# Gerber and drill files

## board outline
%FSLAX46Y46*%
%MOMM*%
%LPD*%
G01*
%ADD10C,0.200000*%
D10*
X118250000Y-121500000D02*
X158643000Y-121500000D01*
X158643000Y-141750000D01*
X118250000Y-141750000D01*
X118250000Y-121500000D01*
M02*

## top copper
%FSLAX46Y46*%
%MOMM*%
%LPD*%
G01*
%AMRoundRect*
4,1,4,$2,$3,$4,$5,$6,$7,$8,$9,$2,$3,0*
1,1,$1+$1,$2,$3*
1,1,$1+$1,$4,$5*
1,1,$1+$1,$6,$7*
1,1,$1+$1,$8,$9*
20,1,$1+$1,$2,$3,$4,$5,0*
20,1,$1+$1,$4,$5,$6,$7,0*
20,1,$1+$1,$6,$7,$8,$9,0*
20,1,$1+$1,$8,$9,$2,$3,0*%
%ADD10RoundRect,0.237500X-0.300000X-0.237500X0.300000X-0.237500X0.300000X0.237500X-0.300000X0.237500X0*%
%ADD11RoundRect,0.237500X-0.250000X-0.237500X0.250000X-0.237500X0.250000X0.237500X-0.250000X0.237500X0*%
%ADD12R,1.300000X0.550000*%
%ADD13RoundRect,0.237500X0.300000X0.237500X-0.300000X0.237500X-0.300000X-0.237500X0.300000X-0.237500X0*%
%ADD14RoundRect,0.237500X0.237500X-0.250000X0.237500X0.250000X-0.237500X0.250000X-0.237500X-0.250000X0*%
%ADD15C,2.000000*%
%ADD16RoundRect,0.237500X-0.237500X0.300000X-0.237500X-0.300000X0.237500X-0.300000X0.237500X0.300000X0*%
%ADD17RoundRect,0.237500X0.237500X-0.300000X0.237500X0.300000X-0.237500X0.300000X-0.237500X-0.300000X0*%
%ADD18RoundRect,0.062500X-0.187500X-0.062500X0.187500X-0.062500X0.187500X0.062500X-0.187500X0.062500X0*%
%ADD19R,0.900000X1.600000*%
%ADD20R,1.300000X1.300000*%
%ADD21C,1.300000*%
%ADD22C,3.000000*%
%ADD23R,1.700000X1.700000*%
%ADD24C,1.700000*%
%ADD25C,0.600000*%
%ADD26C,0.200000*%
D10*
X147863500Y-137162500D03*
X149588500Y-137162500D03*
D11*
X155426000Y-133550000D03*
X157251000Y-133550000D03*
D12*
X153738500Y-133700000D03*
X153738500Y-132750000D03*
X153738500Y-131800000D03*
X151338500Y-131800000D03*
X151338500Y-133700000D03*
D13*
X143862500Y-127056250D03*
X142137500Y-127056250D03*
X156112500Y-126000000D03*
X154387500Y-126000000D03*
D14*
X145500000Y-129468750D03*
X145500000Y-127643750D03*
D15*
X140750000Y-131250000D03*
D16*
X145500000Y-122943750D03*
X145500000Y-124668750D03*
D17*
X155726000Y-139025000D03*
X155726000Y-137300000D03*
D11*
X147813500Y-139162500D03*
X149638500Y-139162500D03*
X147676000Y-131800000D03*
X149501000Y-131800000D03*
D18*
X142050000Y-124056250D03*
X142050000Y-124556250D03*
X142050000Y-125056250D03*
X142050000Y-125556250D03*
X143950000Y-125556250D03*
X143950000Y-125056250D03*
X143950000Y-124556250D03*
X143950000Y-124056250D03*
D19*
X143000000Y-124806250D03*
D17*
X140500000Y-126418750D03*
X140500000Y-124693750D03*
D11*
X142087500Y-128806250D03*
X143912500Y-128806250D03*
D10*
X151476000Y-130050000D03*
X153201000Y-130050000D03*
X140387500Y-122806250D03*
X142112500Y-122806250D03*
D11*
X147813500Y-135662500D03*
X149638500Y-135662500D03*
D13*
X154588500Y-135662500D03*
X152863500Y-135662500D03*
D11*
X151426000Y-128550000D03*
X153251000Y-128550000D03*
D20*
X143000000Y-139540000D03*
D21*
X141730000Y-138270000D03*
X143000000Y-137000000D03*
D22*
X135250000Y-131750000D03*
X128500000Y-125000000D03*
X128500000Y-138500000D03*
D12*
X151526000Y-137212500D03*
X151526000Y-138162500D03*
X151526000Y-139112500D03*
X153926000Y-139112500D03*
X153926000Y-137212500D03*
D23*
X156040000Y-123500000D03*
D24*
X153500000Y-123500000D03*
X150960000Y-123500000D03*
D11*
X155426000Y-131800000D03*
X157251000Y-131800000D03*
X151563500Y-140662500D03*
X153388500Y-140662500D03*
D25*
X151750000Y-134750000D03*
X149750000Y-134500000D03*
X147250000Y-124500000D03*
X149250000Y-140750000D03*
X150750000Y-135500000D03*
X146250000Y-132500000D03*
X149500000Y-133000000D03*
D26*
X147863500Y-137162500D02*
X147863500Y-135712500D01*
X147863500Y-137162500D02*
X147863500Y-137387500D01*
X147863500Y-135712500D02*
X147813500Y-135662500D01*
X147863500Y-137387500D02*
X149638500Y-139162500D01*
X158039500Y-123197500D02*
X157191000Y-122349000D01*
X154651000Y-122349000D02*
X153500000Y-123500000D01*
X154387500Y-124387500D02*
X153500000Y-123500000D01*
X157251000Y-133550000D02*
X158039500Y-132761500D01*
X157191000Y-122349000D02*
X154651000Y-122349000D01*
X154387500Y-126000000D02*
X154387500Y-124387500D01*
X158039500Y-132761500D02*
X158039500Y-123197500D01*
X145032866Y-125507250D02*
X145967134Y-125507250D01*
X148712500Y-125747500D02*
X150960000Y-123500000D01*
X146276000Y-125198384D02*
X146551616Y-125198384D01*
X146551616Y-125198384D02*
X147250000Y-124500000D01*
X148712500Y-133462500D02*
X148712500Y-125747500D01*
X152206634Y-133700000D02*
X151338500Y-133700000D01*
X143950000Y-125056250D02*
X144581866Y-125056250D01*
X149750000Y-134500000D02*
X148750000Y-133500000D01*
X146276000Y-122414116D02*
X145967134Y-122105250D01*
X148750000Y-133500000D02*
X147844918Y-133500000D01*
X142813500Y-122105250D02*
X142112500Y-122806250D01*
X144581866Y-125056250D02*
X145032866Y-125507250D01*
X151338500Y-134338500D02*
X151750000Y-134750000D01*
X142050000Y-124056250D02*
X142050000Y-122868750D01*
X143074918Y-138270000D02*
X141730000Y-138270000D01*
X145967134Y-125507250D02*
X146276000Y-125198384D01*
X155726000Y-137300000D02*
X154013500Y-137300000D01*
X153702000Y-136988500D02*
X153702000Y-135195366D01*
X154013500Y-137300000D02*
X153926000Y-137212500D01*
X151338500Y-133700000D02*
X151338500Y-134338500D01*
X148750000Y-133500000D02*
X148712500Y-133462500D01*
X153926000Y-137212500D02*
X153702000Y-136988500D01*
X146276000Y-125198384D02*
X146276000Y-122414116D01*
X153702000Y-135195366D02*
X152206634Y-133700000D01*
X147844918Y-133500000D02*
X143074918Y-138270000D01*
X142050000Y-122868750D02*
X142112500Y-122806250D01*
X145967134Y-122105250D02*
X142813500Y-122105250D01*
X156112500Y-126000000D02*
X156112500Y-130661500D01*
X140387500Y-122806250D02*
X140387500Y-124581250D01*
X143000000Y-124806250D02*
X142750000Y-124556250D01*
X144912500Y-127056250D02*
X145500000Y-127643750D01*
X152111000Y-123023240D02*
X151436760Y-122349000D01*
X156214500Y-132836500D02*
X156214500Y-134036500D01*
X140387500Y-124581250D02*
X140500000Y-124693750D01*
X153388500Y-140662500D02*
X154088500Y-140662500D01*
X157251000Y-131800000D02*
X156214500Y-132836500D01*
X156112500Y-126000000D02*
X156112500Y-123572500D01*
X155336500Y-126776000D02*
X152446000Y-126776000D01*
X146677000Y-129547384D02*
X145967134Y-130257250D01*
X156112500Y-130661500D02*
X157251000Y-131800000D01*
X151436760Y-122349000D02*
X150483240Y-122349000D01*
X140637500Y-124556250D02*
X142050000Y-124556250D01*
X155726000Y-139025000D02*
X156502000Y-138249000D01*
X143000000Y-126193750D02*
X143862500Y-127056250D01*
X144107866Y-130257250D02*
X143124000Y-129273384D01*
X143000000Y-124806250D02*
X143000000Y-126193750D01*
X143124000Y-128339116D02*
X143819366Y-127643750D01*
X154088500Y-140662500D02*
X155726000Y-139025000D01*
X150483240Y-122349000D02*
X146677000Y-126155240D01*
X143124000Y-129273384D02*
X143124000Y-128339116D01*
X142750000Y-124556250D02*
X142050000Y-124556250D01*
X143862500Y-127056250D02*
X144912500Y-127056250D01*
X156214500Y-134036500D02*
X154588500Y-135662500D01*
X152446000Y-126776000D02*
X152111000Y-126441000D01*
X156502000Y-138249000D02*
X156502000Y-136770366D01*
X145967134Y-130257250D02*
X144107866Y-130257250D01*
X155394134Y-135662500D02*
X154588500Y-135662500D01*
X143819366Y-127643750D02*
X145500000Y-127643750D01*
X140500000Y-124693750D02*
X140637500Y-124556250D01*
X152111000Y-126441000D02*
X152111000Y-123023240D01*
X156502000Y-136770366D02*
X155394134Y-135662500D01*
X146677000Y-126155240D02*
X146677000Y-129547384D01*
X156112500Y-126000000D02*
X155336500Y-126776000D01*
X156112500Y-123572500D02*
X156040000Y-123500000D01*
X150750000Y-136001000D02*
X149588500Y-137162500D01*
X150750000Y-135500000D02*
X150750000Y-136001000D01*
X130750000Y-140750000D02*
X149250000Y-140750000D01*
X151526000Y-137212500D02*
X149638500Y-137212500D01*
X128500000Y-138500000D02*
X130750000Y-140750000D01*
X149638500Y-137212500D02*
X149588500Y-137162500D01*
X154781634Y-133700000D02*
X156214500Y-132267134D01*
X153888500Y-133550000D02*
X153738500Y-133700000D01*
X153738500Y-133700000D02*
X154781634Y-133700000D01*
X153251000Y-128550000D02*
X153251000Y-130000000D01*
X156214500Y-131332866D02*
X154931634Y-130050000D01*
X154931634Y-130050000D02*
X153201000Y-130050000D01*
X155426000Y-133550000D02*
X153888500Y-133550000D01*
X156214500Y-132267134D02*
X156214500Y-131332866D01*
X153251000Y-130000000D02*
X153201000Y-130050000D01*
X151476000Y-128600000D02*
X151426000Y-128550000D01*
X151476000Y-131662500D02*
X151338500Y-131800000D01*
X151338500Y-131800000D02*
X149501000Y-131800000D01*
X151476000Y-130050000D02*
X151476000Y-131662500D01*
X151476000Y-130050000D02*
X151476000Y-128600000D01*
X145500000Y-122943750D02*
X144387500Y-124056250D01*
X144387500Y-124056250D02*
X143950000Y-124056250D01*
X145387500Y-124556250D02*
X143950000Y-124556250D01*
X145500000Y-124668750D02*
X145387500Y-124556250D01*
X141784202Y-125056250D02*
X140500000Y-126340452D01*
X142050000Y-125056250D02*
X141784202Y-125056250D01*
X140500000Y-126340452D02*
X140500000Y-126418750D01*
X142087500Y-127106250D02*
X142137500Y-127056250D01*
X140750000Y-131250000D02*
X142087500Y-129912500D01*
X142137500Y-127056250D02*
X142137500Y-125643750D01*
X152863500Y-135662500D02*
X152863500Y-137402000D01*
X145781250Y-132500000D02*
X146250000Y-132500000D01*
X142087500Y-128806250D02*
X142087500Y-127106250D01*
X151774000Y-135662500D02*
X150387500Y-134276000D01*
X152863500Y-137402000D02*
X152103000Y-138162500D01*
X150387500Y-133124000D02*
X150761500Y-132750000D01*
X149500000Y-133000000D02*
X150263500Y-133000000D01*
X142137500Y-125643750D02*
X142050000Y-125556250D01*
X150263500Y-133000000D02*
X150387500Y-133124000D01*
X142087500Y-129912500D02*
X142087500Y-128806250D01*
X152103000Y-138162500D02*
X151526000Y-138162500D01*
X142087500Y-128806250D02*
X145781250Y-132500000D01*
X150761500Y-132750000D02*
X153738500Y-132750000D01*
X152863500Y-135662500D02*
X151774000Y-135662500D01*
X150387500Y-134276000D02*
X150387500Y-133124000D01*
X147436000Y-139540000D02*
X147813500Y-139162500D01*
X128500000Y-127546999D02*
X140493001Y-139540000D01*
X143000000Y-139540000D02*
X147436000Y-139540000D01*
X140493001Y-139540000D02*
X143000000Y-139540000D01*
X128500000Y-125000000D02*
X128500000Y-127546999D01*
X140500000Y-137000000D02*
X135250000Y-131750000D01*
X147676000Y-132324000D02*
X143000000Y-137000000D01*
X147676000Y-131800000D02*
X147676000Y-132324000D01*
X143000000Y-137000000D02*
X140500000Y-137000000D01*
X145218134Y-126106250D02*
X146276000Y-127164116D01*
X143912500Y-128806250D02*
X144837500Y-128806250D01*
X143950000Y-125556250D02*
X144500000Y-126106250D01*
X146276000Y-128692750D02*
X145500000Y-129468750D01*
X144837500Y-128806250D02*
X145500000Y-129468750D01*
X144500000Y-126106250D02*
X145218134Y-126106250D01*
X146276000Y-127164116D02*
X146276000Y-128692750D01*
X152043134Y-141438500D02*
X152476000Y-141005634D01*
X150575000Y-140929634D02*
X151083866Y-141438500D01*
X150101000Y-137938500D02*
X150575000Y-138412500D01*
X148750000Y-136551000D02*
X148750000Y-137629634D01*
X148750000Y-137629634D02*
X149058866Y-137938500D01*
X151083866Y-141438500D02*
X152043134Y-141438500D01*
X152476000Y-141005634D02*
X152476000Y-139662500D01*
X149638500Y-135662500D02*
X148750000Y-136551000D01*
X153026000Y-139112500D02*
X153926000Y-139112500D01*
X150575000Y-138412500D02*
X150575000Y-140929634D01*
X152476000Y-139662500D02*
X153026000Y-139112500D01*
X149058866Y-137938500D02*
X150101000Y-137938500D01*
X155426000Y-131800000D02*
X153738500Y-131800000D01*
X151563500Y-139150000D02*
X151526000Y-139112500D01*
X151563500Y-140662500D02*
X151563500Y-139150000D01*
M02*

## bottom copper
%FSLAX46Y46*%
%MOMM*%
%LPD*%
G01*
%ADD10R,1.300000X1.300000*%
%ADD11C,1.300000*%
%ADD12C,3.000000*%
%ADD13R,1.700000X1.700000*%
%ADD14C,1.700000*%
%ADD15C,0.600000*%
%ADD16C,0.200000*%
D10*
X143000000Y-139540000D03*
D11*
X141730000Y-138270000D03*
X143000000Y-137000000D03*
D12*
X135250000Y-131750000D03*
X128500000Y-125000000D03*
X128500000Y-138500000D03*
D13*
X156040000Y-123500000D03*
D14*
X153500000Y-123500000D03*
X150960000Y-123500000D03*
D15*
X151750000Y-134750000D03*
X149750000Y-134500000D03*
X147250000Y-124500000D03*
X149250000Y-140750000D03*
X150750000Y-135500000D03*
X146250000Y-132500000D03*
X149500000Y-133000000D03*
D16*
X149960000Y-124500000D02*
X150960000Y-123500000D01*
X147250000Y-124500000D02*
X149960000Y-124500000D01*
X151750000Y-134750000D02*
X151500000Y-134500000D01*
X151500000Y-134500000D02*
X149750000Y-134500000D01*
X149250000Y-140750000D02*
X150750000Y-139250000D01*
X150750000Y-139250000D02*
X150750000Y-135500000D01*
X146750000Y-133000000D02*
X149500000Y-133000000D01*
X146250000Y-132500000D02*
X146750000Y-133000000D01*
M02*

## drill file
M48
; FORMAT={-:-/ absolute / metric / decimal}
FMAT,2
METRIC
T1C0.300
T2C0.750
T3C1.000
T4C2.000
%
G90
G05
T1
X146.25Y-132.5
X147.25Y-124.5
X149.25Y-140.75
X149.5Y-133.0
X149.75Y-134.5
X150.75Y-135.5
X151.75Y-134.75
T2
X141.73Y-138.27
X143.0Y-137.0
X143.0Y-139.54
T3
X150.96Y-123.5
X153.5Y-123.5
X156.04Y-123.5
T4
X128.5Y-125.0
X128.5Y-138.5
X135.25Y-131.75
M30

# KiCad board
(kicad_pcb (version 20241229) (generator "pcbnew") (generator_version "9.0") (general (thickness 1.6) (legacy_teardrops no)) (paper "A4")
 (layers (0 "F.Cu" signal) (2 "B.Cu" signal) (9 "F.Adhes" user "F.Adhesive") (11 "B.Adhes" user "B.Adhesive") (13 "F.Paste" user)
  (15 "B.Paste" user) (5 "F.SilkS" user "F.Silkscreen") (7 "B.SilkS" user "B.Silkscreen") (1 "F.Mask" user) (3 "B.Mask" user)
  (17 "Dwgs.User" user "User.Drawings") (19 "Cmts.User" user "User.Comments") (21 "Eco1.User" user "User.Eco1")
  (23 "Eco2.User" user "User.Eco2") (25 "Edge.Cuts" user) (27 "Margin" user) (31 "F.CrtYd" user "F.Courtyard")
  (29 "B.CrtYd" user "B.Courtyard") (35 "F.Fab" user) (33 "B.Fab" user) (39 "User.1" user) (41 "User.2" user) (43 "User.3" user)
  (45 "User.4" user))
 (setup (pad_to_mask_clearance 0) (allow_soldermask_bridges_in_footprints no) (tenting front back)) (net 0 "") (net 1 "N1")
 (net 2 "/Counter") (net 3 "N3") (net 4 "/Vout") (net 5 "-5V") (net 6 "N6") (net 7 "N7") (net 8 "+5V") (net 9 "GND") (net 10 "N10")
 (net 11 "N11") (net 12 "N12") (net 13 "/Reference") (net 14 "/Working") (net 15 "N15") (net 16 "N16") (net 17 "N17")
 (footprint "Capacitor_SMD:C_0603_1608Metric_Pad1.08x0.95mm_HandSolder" (layer "F.Cu") (at 148.726 137.1625)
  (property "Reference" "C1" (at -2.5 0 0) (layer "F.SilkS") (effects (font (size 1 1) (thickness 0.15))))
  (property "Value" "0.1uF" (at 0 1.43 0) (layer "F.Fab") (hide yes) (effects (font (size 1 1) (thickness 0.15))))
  (pad "1" smd roundrect (at -0.8625 0) (size 1.075 0.95) (layers "F.Cu" "F.Mask" "F.Paste") (roundrect_rratio 0.25) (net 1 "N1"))
  (pad "2" smd roundrect (at 0.8625 0) (size 1.075 0.95) (layers "F.Cu" "F.Mask" "F.Paste") (roundrect_rratio 0.25) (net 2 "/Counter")))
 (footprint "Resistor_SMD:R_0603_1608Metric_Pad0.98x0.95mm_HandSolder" (layer "F.Cu") (at 156.3385 133.55)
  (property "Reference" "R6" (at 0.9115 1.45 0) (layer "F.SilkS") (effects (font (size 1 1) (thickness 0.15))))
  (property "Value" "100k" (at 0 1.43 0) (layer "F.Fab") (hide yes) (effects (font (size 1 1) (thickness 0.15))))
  (pad "1" smd roundrect (at -0.9125 0) (size 0.975 0.95) (layers "F.Cu" "F.Mask" "F.Paste") (roundrect_rratio 0.25) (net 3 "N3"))
  (pad "2" smd roundrect (at 0.9125 0) (size 0.975 0.95) (layers "F.Cu" "F.Mask" "F.Paste") (roundrect_rratio 0.25) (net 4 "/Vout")))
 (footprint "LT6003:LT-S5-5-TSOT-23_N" (layer "F.Cu") (at 152.5385 132.75 180)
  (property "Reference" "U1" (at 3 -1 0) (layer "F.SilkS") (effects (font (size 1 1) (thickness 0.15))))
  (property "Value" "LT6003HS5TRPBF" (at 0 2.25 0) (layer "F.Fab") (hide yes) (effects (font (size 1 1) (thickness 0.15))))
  (pad "1" smd rect (at -1.2 -0.95 270) (size 0.55 1.3) (layers "F.Cu" "F.Mask" "F.Paste") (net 3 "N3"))
  (pad "2" smd rect (at -1.2 0 270) (size 0.55 1.3) (layers "F.Cu" "F.Mask" "F.Paste") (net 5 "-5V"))
  (pad "3" smd rect (at -1.2 0.95 270) (size 0.55 1.3) (layers "F.Cu" "F.Mask" "F.Paste") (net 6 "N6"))
  (pad "4" smd rect (at 1.2 0.95 270) (size 0.55 1.3) (layers "F.Cu" "F.Mask" "F.Paste") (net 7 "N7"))
  (pad "5" smd rect (at 1.2 -0.95 270) (size 0.55 1.3) (layers "F.Cu" "F.Mask" "F.Paste") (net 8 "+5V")))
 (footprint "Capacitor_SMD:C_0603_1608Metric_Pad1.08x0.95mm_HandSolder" (layer "F.Cu") (at 143 127.05625 180)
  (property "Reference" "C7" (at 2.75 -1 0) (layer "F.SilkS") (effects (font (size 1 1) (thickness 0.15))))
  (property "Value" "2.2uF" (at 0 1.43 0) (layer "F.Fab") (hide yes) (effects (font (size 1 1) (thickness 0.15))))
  (pad "1" smd roundrect (at -0.8625 0 180) (size 1.075 0.95) (layers "F.Cu" "F.Mask" "F.Paste") (roundrect_rratio 0.25) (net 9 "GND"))
  (pad "2" smd roundrect (at 0.8625 0 180) (size 1.075 0.95) (layers "F.Cu" "F.Mask" "F.Paste") (roundrect_rratio 0.25) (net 5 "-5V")))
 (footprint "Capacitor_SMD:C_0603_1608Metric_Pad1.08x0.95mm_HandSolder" (layer "F.Cu") (at 155.25 126 180)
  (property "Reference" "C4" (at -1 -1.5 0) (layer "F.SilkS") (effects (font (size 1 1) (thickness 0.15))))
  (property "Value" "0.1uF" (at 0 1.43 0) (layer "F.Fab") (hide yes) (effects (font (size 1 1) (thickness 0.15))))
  (pad "1" smd roundrect (at -0.8625 0 180) (size 1.075 0.95) (layers "F.Cu" "F.Mask" "F.Paste") (roundrect_rratio 0.25) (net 9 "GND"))
  (pad "2" smd roundrect (at 0.8625 0 180) (size 1.075 0.95) (layers "F.Cu" "F.Mask" "F.Paste") (roundrect_rratio 0.25) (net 4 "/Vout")))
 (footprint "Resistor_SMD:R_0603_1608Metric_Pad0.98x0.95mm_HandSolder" (layer "F.Cu") (at 145.5 128.55625 90)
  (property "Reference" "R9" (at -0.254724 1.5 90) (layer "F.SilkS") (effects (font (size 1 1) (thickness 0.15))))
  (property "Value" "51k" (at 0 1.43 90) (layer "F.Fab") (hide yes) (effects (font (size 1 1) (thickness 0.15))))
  (pad "1" smd roundrect (at -0.9125 0 90) (size 0.975 0.95) (layers "F.Cu" "F.Mask" "F.Paste") (roundrect_rratio 0.25) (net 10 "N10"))
  (pad "2" smd roundrect (at 0.9125 0 90) (size 0.975 0.95) (layers "F.Cu" "F.Mask" "F.Paste") (roundrect_rratio 0.25) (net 9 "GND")))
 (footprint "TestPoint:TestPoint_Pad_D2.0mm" (layer "F.Cu") (at 140.75 131.25)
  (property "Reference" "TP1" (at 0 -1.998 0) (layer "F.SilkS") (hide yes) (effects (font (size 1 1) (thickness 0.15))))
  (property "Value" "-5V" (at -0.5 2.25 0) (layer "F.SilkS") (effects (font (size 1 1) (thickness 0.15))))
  (pad "1" smd circle (at 0 0) (size 2 2) (layers "F.Cu" "F.Mask") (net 5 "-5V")))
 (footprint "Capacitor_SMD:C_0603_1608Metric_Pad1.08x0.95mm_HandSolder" (layer "F.Cu") (at 145.5 123.80625 -90)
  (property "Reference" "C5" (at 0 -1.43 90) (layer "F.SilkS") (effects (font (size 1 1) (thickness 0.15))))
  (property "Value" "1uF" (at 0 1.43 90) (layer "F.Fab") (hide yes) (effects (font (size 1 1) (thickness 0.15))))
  (pad "1" smd roundrect (at -0.8625 0 270) (size 1.075 0.95) (layers "F.Cu" "F.Mask" "F.Paste") (roundrect_rratio 0.25) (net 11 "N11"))
  (pad "2" smd roundrect (at 0.8625 0 270) (size 1.075 0.95) (layers "F.Cu" "F.Mask" "F.Paste") (roundrect_rratio 0.25) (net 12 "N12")))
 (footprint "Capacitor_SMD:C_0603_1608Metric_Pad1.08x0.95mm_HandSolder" (layer "F.Cu") (at 155.726 138.1625 90)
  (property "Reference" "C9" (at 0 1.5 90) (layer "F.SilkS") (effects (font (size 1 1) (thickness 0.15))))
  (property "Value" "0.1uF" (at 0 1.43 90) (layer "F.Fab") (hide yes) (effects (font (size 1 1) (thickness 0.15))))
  (pad "1" smd roundrect (at -0.8625 0 90) (size 1.075 0.95) (layers "F.Cu" "F.Mask" "F.Paste") (roundrect_rratio 0.25) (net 9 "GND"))
  (pad "2" smd roundrect (at 0.8625 0 90) (size 1.075 0.95) (layers "F.Cu" "F.Mask" "F.Paste") (roundrect_rratio 0.25) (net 8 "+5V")))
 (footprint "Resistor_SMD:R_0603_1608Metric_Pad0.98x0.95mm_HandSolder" (layer "F.Cu") (at 148.726 139.1625)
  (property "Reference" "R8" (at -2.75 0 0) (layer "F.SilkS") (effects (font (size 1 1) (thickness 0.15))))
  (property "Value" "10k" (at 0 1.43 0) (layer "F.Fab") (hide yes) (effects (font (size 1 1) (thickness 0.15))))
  (pad "1" smd roundrect (at -0.9125 0) (size 0.975 0.95) (layers "F.Cu" "F.Mask" "F.Paste") (roundrect_rratio 0.25) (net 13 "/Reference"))
  (pad "2" smd roundrect (at 0.9125 0) (size 0.975 0.95) (layers "F.Cu" "F.Mask" "F.Paste") (roundrect_rratio 0.25) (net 1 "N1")))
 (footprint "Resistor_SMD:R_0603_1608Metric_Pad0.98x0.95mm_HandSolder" (layer "F.Cu") (at 148.5885 131.8)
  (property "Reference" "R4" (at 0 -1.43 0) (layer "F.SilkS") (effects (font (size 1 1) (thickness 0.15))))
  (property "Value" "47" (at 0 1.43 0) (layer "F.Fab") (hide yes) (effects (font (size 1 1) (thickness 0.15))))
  (pad "1" smd roundrect (at -0.9125 0) (size 0.975 0.95) (layers "F.Cu" "F.Mask" "F.Paste") (roundrect_rratio 0.25) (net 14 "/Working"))
  (pad "2" smd roundrect (at 0.9125 0) (size 0.975 0.95) (layers "F.Cu" "F.Mask" "F.Paste") (roundrect_rratio 0.25) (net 7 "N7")))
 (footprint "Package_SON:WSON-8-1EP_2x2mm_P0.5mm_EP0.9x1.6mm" (layer "F.Cu") (at 143 124.80625)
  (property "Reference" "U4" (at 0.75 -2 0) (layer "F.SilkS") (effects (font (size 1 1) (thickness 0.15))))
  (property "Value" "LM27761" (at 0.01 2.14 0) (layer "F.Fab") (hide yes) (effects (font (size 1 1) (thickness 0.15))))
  (pad "" smd rect (at 0 -0.4) (size 0.75 0.65) (layers "F.Paste"))
  (pad "" smd rect (at 0 0.4) (size 0.75 0.65) (layers "F.Paste"))
  (pad "1" smd roundrect (at -0.95 -0.75) (size 0.5 0.25) (layers "F.Cu" "F.Mask" "F.Paste") (roundrect_rratio 0.25) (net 8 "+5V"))
  (pad "2" smd roundrect (at -0.95 -0.25) (size 0.5 0.25) (layers "F.Cu" "F.Mask" "F.Paste") (roundrect_rratio 0.25) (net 9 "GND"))
  (pad "3" smd roundrect (at -0.95 0.25) (size 0.5 0.25) (layers "F.Cu" "F.Mask" "F.Paste") (roundrect_rratio 0.25) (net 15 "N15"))
  (pad "4" smd roundrect (at -0.95 0.75) (size 0.5 0.25) (layers "F.Cu" "F.Mask" "F.Paste") (roundrect_rratio 0.25) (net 5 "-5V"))
  (pad "5" smd roundrect (at 0.95 0.75) (size 0.5 0.25) (layers "F.Cu" "F.Mask" "F.Paste") (roundrect_rratio 0.25) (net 10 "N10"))
  (pad "6" smd roundrect (at 0.95 0.25) (size 0.5 0.25) (layers "F.Cu" "F.Mask" "F.Paste") (roundrect_rratio 0.25) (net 8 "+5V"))
  (pad "7" smd roundrect (at 0.95 -0.25) (size 0.5 0.25) (layers "F.Cu" "F.Mask" "F.Paste") (roundrect_rratio 0.25) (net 12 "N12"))
  (pad "8" smd roundrect (at 0.95 -0.75) (size 0.5 0.25) (layers "F.Cu" "F.Mask" "F.Paste") (roundrect_rratio 0.25) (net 11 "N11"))
  (pad "9" smd rect (at 0 0) (size 0.9 1.6) (layers "F.Cu" "F.Mask") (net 9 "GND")))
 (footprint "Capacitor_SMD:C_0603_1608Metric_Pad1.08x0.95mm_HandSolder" (layer "F.Cu") (at 140.5 125.55625 90)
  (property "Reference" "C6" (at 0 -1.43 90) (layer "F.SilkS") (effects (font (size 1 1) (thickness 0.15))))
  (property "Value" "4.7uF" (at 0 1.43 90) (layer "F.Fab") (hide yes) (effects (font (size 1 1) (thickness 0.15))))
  (pad "1" smd roundrect (at -0.8625 0 90) (size 1.075 0.95) (layers "F.Cu" "F.Mask" "F.Paste") (roundrect_rratio 0.25) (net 15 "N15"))
  (pad "2" smd roundrect (at 0.8625 0 90) (size 1.075 0.95) (layers "F.Cu" "F.Mask" "F.Paste") (roundrect_rratio 0.25) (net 9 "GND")))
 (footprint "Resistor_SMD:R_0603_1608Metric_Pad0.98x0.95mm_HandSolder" (layer "F.Cu") (at 143 128.80625)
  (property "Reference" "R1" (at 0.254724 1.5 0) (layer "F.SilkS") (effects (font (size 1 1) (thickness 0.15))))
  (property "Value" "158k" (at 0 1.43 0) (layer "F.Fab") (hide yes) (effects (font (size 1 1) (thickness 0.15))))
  (pad "1" smd roundrect (at -0.9125 0) (size 0.975 0.95) (layers "F.Cu" "F.Mask" "F.Paste") (roundrect_rratio 0.25) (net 5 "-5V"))
  (pad "2" smd roundrect (at 0.9125 0) (size 0.975 0.95) (layers "F.Cu" "F.Mask" "F.Paste") (roundrect_rratio 0.25) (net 10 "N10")))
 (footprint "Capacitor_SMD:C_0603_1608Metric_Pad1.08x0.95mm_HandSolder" (layer "F.Cu") (at 152.3385 130.05)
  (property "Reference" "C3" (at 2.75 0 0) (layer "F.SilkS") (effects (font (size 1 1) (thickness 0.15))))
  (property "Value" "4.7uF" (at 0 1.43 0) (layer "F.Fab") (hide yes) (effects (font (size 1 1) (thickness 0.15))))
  (pad "1" smd roundrect (at -0.8625 0) (size 1.075 0.95) (layers "F.Cu" "F.Mask" "F.Paste") (roundrect_rratio 0.25) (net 7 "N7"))
  (pad "2" smd roundrect (at 0.8625 0) (size 1.075 0.95) (layers "F.Cu" "F.Mask" "F.Paste") (roundrect_rratio 0.25) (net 3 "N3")))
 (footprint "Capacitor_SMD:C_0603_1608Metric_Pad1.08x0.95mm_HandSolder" (layer "F.Cu") (at 141.25 122.80625)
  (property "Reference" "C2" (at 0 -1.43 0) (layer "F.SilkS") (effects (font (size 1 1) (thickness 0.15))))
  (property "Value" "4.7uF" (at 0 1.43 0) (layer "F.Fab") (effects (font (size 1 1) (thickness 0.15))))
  (pad "1" smd roundrect (at -0.8625 0) (size 1.075 0.95) (layers "F.Cu" "F.Mask" "F.Paste") (roundrect_rratio 0.25) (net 9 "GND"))
  (pad "2" smd roundrect (at 0.8625 0) (size 1.075 0.95) (layers "F.Cu" "F.Mask" "F.Paste") (roundrect_rratio 0.25) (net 8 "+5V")))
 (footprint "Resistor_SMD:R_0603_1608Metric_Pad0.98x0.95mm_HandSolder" (layer "F.Cu") (at 148.726 135.6625)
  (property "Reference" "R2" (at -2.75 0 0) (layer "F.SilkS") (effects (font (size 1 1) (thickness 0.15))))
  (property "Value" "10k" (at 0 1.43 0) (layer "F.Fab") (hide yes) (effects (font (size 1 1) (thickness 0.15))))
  (pad "1" smd roundrect (at -0.9125 0) (size 0.975 0.95) (layers "F.Cu" "F.Mask" "F.Paste") (roundrect_rratio 0.25) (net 1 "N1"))
  (pad "2" smd roundrect (at 0.9125 0) (size 0.975 0.95) (layers "F.Cu" "F.Mask" "F.Paste") (roundrect_rratio 0.25) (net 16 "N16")))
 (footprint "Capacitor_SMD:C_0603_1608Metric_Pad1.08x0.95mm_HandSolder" (layer "F.Cu") (at 153.726 135.6625 180)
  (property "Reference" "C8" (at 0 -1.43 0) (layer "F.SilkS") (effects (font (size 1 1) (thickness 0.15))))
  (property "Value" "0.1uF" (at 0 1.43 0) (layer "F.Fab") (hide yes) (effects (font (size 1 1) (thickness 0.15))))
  (pad "1" smd roundrect (at -0.8625 0 180) (size 1.075 0.95) (layers "F.Cu" "F.Mask" "F.Paste") (roundrect_rratio 0.25) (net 9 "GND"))
  (pad "2" smd roundrect (at 0.8625 0 180) (size 1.075 0.95) (layers "F.Cu" "F.Mask" "F.Paste") (roundrect_rratio 0.25) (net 5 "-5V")))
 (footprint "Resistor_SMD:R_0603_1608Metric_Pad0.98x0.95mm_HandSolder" (layer "F.Cu") (at 152.3385 128.55)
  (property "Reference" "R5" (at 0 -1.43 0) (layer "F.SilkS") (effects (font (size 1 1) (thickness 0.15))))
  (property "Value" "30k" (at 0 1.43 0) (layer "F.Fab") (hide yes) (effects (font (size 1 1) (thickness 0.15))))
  (pad "1" smd roundrect (at -0.9125 0) (size 0.975 0.95) (layers "F.Cu" "F.Mask" "F.Paste") (roundrect_rratio 0.25) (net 7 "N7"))
  (pad "2" smd roundrect (at 0.9125 0) (size 0.975 0.95) (layers "F.Cu" "F.Mask" "F.Paste") (roundrect_rratio 0.25) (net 3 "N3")))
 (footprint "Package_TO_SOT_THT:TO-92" (layer "F.Cu") (at 143 139.54 90)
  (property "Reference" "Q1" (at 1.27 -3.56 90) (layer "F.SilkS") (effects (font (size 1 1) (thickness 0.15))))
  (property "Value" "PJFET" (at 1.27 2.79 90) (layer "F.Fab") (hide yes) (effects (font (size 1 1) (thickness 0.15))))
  (pad "1" thru_hole rect (at 0 0 90) (size 1.3 1.3) (drill 0.75) (layers "*.Cu" "*.Mask") (remove_unused_layers no) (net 13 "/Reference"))
  (pad "2" thru_hole circle (at 1.27 -1.27 90) (size 1.3 1.3) (drill 0.75) (layers "*.Cu" "*.Mask") (remove_unused_layers no) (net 8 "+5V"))
  (pad "3" thru_hole circle (at 2.54 0 90) (size 1.3 1.3) (drill 0.75) (layers "*.Cu" "*.Mask") (remove_unused_layers no)
   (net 14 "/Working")))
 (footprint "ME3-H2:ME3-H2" (layer "F.Cu") (at 128.5 131.75 -90)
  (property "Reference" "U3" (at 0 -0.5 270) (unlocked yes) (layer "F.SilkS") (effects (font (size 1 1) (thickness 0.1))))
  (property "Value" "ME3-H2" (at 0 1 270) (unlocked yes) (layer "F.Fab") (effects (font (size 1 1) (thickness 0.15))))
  (pad "1" thru_hole circle (at 0 -6.75 270) (size 3 3) (drill 2) (layers "*.Cu" "*.Mask") (remove_unused_layers no) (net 14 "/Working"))
  (pad "2" thru_hole circle (at -6.75 0 270) (size 3 3) (drill 2) (layers "*.Cu" "*.Mask") (remove_unused_layers no) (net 13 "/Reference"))
  (pad "3" thru_hole circle (at 6.75 0 270) (size 3 3) (drill 2) (layers "*.Cu" "*.Mask") (remove_unused_layers no) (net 2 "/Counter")))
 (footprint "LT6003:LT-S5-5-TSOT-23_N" (layer "F.Cu") (at 152.726 138.1625)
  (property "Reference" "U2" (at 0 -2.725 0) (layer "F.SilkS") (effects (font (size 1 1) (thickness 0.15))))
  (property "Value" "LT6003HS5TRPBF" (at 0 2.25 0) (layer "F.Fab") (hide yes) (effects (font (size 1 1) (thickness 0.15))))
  (pad "1" smd rect (at -1.2 -0.95 90) (size 0.55 1.3) (layers "F.Cu" "F.Mask" "F.Paste") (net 2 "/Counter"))
  (pad "2" smd rect (at -1.2 0 90) (size 0.55 1.3) (layers "F.Cu" "F.Mask" "F.Paste") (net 5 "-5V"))
  (pad "3" smd rect (at -1.2 0.95 90) (size 0.55 1.3) (layers "F.Cu" "F.Mask" "F.Paste") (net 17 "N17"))
  (pad "4" smd rect (at 1.2 0.95 90) (size 0.55 1.3) (layers "F.Cu" "F.Mask" "F.Paste") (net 16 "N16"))
  (pad "5" smd rect (at 1.2 -0.95 90) (size 0.55 1.3) (layers "F.Cu" "F.Mask" "F.Paste") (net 8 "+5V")))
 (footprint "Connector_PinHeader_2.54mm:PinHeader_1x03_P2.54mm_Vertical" (layer "F.Cu") (at 156.04 123.5 -90)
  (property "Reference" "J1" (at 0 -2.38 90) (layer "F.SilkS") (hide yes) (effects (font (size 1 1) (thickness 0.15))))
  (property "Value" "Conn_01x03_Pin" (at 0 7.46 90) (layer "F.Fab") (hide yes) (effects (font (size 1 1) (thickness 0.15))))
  (pad "1" thru_hole rect (at 0 0 270) (size 1.7 1.7) (drill 1) (layers "*.Cu" "*.Mask") (remove_unused_layers no) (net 9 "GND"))
  (pad "2" thru_hole circle (at 0 2.54 270) (size 1.7 1.7) (drill 1) (layers "*.Cu" "*.Mask") (remove_unused_layers no) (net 4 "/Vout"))
  (pad "3" thru_hole circle (at 0 5.08 270) (size 1.7 1.7) (drill 1) (layers "*.Cu" "*.Mask") (remove_unused_layers no) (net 8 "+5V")))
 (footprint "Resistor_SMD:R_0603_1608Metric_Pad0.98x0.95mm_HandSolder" (layer "F.Cu") (at 156.3385 131.8)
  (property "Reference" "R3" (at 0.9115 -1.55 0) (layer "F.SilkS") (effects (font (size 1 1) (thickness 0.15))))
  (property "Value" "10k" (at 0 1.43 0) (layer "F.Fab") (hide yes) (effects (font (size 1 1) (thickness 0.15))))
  (pad "1" smd roundrect (at -0.9125 0) (size 0.975 0.95) (layers "F.Cu" "F.Mask" "F.Paste") (roundrect_rratio 0.25) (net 6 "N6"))
  (pad "2" smd roundrect (at 0.9125 0) (size 0.975 0.95) (layers "F.Cu" "F.Mask" "F.Paste") (roundrect_rratio 0.25) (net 9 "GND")))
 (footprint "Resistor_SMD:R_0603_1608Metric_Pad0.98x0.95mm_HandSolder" (layer "F.Cu") (at 152.476 140.6625)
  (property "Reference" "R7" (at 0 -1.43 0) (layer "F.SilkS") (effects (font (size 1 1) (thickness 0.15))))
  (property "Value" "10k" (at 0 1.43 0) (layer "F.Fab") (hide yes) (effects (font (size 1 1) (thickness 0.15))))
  (pad "1" smd roundrect (at -0.9125 0) (size 0.975 0.95) (layers "F.Cu" "F.Mask" "F.Paste") (roundrect_rratio 0.25) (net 17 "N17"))
  (pad "2" smd roundrect (at 0.9125 0) (size 0.975 0.95) (layers "F.Cu" "F.Mask" "F.Paste") (roundrect_rratio 0.25) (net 9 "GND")))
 (gr_rect (start 118.25 121.5) (end 158.643 141.75) (stroke (width 0.2) (type solid)) (fill no) (layer "Edge.Cuts"))
 (segment (start 147.8635 137.1625) (end 147.8635 135.7125) (width 0.2) (layer "F.Cu") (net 1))
 (segment (start 147.8635 137.1625) (end 147.8635 137.3875) (width 0.2) (layer "F.Cu") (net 1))
 (segment (start 147.8635 135.7125) (end 147.8135 135.6625) (width 0.2) (layer "F.Cu") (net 1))
 (segment (start 147.8635 137.3875) (end 149.6385 139.1625) (width 0.2) (layer "F.Cu") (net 1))
 (segment (start 158.0395 123.1975) (end 157.191 122.349) (width 0.2) (layer "F.Cu") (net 4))
 (segment (start 154.651 122.349) (end 153.5 123.5) (width 0.2) (layer "F.Cu") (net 4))
 (segment (start 154.3875 124.3875) (end 153.5 123.5) (width 0.2) (layer "F.Cu") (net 4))
 (segment (start 157.251 133.55) (end 158.0395 132.7615) (width 0.2) (layer "F.Cu") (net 4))
 (segment (start 157.191 122.349) (end 154.651 122.349) (width 0.2) (layer "F.Cu") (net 4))
 (segment (start 154.3875 126) (end 154.3875 124.3875) (width 0.2) (layer "F.Cu") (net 4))
 (segment (start 158.0395 132.7615) (end 158.0395 123.1975) (width 0.2) (layer "F.Cu") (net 4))
 (segment (start 145.032866 125.50725) (end 145.967134 125.50725) (width 0.2) (layer "F.Cu") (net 8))
 (segment (start 148.7125 125.7475) (end 150.96 123.5) (width 0.2) (layer "F.Cu") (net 8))
 (segment (start 146.276 125.198384) (end 146.551616 125.198384) (width 0.2) (layer "F.Cu") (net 8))
 (segment (start 146.551616 125.198384) (end 147.25 124.5) (width 0.2) (layer "F.Cu") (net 8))
 (segment (start 148.7125 133.4625) (end 148.7125 125.7475) (width 0.2) (layer "F.Cu") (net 8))
 (segment (start 152.206634 133.7) (end 151.3385 133.7) (width 0.2) (layer "F.Cu") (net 8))
 (segment (start 143.95 125.05625) (end 144.581866 125.05625) (width 0.2) (layer "F.Cu") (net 8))
 (segment (start 149.75 134.5) (end 148.75 133.5) (width 0.2) (layer "F.Cu") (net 8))
 (segment (start 146.276 122.414116) (end 145.967134 122.10525) (width 0.2) (layer "F.Cu") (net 8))
 (segment (start 148.75 133.5) (end 147.844918 133.5) (width 0.2) (layer "F.Cu") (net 8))
 (segment (start 142.8135 122.10525) (end 142.1125 122.80625) (width 0.2) (layer "F.Cu") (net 8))
 (segment (start 144.581866 125.05625) (end 145.032866 125.50725) (width 0.2) (layer "F.Cu") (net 8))
 (segment (start 151.3385 134.3385) (end 151.75 134.75) (width 0.2) (layer "F.Cu") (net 8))
 (segment (start 142.05 124.05625) (end 142.05 122.86875) (width 0.2) (layer "F.Cu") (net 8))
 (segment (start 143.074918 138.27) (end 141.73 138.27) (width 0.2) (layer "F.Cu") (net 8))
 (segment (start 145.967134 125.50725) (end 146.276 125.198384) (width 0.2) (layer "F.Cu") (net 8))
 (segment (start 155.726 137.3) (end 154.0135 137.3) (width 0.2) (layer "F.Cu") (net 8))
 (segment (start 153.702 136.9885) (end 153.702 135.195366) (width 0.2) (layer "F.Cu") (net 8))
 (segment (start 154.0135 137.3) (end 153.926 137.2125) (width 0.2) (layer "F.Cu") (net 8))
 (segment (start 151.3385 133.7) (end 151.3385 134.3385) (width 0.2) (layer "F.Cu") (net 8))
 (segment (start 148.75 133.5) (end 148.7125 133.4625) (width 0.2) (layer "F.Cu") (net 8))
 (segment (start 153.926 137.2125) (end 153.702 136.9885) (width 0.2) (layer "F.Cu") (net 8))
 (segment (start 146.276 125.198384) (end 146.276 122.414116) (width 0.2) (layer "F.Cu") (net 8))
 (segment (start 153.702 135.195366) (end 152.206634 133.7) (width 0.2) (layer "F.Cu") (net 8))
 (segment (start 147.844918 133.5) (end 143.074918 138.27) (width 0.2) (layer "F.Cu") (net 8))
 (segment (start 142.05 122.86875) (end 142.1125 122.80625) (width 0.2) (layer "F.Cu") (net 8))
 (segment (start 145.967134 122.10525) (end 142.8135 122.10525) (width 0.2) (layer "F.Cu") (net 8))
 (via (at 151.75 134.75) (size 0.6) (drill 0.3) (layers "F.Cu" "B.Cu") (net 8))
 (via (at 149.75 134.5) (size 0.6) (drill 0.3) (layers "F.Cu" "B.Cu") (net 8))
 (via (at 147.25 124.5) (size 0.6) (drill 0.3) (layers "F.Cu" "B.Cu") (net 8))
 (segment (start 149.96 124.5) (end 150.96 123.5) (width 0.2) (layer "B.Cu") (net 8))
 (segment (start 147.25 124.5) (end 149.96 124.5) (width 0.2) (layer "B.Cu") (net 8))
 (segment (start 151.75 134.75) (end 151.5 134.5) (width 0.2) (layer "B.Cu") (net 8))
 (segment (start 151.5 134.5) (end 149.75 134.5) (width 0.2) (layer "B.Cu") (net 8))
 (segment (start 156.1125 126) (end 156.1125 130.6615) (width 0.2) (layer "F.Cu") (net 9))
 (segment (start 140.3875 122.80625) (end 140.3875 124.58125) (width 0.2) (layer "F.Cu") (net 9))
 (segment (start 143 124.80625) (end 142.75 124.55625) (width 0.2) (layer "F.Cu") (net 9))
 (segment (start 144.9125 127.05625) (end 145.5 127.64375) (width 0.2) (layer "F.Cu") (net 9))
 (segment (start 152.111 123.02324) (end 151.43676 122.349) (width 0.2) (layer "F.Cu") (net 9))
 (segment (start 156.2145 132.8365) (end 156.2145 134.0365) (width 0.2) (layer "F.Cu") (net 9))
 (segment (start 140.3875 124.58125) (end 140.5 124.69375) (width 0.2) (layer "F.Cu") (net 9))
 (segment (start 153.3885 140.6625) (end 154.0885 140.6625) (width 0.2) (layer "F.Cu") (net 9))
 (segment (start 157.251 131.8) (end 156.2145 132.8365) (width 0.2) (layer "F.Cu") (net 9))
 (segment (start 156.1125 126) (end 156.1125 123.5725) (width 0.2) (layer "F.Cu") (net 9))
 (segment (start 155.3365 126.776) (end 152.446 126.776) (width 0.2) (layer "F.Cu") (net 9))
 (segment (start 146.677 129.547384) (end 145.967134 130.25725) (width 0.2) (layer "F.Cu") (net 9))
 (segment (start 156.1125 130.6615) (end 157.251 131.8) (width 0.2) (layer "F.Cu") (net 9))
 (segment (start 151.43676 122.349) (end 150.48324 122.349) (width 0.2) (layer "F.Cu") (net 9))
 (segment (start 140.6375 124.55625) (end 142.05 124.55625) (width 0.2) (layer "F.Cu") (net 9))
 (segment (start 155.726 139.025) (end 156.502 138.249) (width 0.2) (layer "F.Cu") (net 9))
 (segment (start 143 126.19375) (end 143.8625 127.05625) (width 0.2) (layer "F.Cu") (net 9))
 (segment (start 144.107866 130.25725) (end 143.124 129.273384) (width 0.2) (layer "F.Cu") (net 9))
 (segment (start 143 124.80625) (end 143 126.19375) (width 0.2) (layer "F.Cu") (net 9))
 (segment (start 143.124 128.339116) (end 143.819366 127.64375) (width 0.2) (layer "F.Cu") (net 9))
 (segment (start 154.0885 140.6625) (end 155.726 139.025) (width 0.2) (layer "F.Cu") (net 9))
 (segment (start 150.48324 122.349) (end 146.677 126.15524) (width 0.2) (layer "F.Cu") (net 9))
 (segment (start 143.124 129.273384) (end 143.124 128.339116) (width 0.2) (layer "F.Cu") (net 9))
 (segment (start 142.75 124.55625) (end 142.05 124.55625) (width 0.2) (layer "F.Cu") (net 9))
 (segment (start 143.8625 127.05625) (end 144.9125 127.05625) (width 0.2) (layer "F.Cu") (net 9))
 (segment (start 156.2145 134.0365) (end 154.5885 135.6625) (width 0.2) (layer "F.Cu") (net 9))
 (segment (start 152.446 126.776) (end 152.111 126.441) (width 0.2) (layer "F.Cu") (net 9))
 (segment (start 156.502 138.249) (end 156.502 136.770366) (width 0.2) (layer "F.Cu") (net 9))
 (segment (start 145.967134 130.25725) (end 144.107866 130.25725) (width 0.2) (layer "F.Cu") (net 9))
 (segment (start 155.394134 135.6625) (end 154.5885 135.6625) (width 0.2) (layer "F.Cu") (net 9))
 (segment (start 143.819366 127.64375) (end 145.5 127.64375) (width 0.2) (layer "F.Cu") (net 9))
 (segment (start 140.5 124.69375) (end 140.6375 124.55625) (width 0.2) (layer "F.Cu") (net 9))
 (segment (start 152.111 126.441) (end 152.111 123.02324) (width 0.2) (layer "F.Cu") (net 9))
 (segment (start 156.502 136.770366) (end 155.394134 135.6625) (width 0.2) (layer "F.Cu") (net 9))
 (segment (start 146.677 126.15524) (end 146.677 129.547384) (width 0.2) (layer "F.Cu") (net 9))
 (segment (start 156.1125 126) (end 155.3365 126.776) (width 0.2) (layer "F.Cu") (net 9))
 (segment (start 156.1125 123.5725) (end 156.04 123.5) (width 0.2) (layer "F.Cu") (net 9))
 (segment (start 150.75 136.001) (end 149.5885 137.1625) (width 0.2) (layer "F.Cu") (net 2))
 (segment (start 150.75 135.5) (end 150.75 136.001) (width 0.2) (layer "F.Cu") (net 2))
 (segment (start 130.75 140.75) (end 149.25 140.75) (width 0.2) (layer "F.Cu") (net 2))
 (segment (start 151.526 137.2125) (end 149.6385 137.2125) (width 0.2) (layer "F.Cu") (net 2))
 (segment (start 128.5 138.5) (end 130.75 140.75) (width 0.2) (layer "F.Cu") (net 2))
 (segment (start 149.6385 137.2125) (end 149.5885 137.1625) (width 0.2) (layer "F.Cu") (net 2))
 (via (at 149.25 140.75) (size 0.6) (drill 0.3) (layers "F.Cu" "B.Cu") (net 2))
 (via (at 150.75 135.5) (size 0.6) (drill 0.3) (layers "F.Cu" "B.Cu") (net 2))
 (segment (start 149.25 140.75) (end 150.75 139.25) (width 0.2) (layer "B.Cu") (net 2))
 (segment (start 150.75 139.25) (end 150.75 135.5) (width 0.2) (layer "B.Cu") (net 2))
 (segment (start 154.781634 133.7) (end 156.2145 132.267134) (width 0.2) (layer "F.Cu") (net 3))
 (segment (start 153.8885 133.55) (end 153.7385 133.7) (width 0.2) (layer "F.Cu") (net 3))
 (segment (start 153.7385 133.7) (end 154.781634 133.7) (width 0.2) (layer "F.Cu") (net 3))
 (segment (start 153.251 128.55) (end 153.251 130) (width 0.2) (layer "F.Cu") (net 3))
 (segment (start 156.2145 131.332866) (end 154.931634 130.05) (width 0.2) (layer "F.Cu") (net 3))
 (segment (start 154.931634 130.05) (end 153.201 130.05) (width 0.2) (layer "F.Cu") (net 3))
 (segment (start 155.426 133.55) (end 153.8885 133.55) (width 0.2) (layer "F.Cu") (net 3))
 (segment (start 156.2145 132.267134) (end 156.2145 131.332866) (width 0.2) (layer "F.Cu") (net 3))
 (segment (start 153.251 130) (end 153.201 130.05) (width 0.2) (layer "F.Cu") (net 3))
 (segment (start 151.476 128.6) (end 151.426 128.55) (width 0.2) (layer "F.Cu") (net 7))
 (segment (start 151.476 131.6625) (end 151.3385 131.8) (width 0.2) (layer "F.Cu") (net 7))
 (segment (start 151.3385 131.8) (end 149.501 131.8) (width 0.2) (layer "F.Cu") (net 7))
 (segment (start 151.476 130.05) (end 151.476 131.6625) (width 0.2) (layer "F.Cu") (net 7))
 (segment (start 151.476 130.05) (end 151.476 128.6) (width 0.2) (layer "F.Cu") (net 7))
 (segment (start 145.5 122.94375) (end 144.3875 124.05625) (width 0.2) (layer "F.Cu") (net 11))
 (segment (start 144.3875 124.05625) (end 143.95 124.05625) (width 0.2) (layer "F.Cu") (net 11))
 (segment (start 145.3875 124.55625) (end 143.95 124.55625) (width 0.2) (layer "F.Cu") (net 12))
 (segment (start 145.5 124.66875) (end 145.3875 124.55625) (width 0.2) (layer "F.Cu") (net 12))
 (segment (start 141.784202 125.05625) (end 140.5 126.340452) (width 0.2) (layer "F.Cu") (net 15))
 (segment (start 142.05 125.05625) (end 141.784202 125.05625) (width 0.2) (layer "F.Cu") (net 15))
 (segment (start 140.5 126.340452) (end 140.5 126.41875) (width 0.2) (layer "F.Cu") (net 15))
 (segment (start 142.0875 127.10625) (end 142.1375 127.05625) (width 0.2) (layer "F.Cu") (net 5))
 (segment (start 140.75 131.25) (end 142.0875 129.9125) (width 0.2) (layer "F.Cu") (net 5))
 (segment (start 142.1375 127.05625) (end 142.1375 125.64375) (width 0.2) (layer "F.Cu") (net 5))
 (segment (start 152.8635 135.6625) (end 152.8635 137.402) (width 0.2) (layer "F.Cu") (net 5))
 (segment (start 145.78125 132.5) (end 146.25 132.5) (width 0.2) (layer "F.Cu") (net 5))
 (segment (start 142.0875 128.80625) (end 142.0875 127.10625) (width 0.2) (layer "F.Cu") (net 5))
 (segment (start 151.774 135.6625) (end 150.3875 134.276) (width 0.2) (layer "F.Cu") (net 5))
 (segment (start 152.8635 137.402) (end 152.103 138.1625) (width 0.2) (layer "F.Cu") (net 5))
 (segment (start 150.3875 133.124) (end 150.7615 132.75) (width 0.2) (layer "F.Cu") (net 5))
 (segment (start 149.5 133) (end 150.2635 133) (width 0.2) (layer "F.Cu") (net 5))
 (segment (start 142.1375 125.64375) (end 142.05 125.55625) (width 0.2) (layer "F.Cu") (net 5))
 (segment (start 150.2635 133) (end 150.3875 133.124) (width 0.2) (layer "F.Cu") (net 5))
 (segment (start 142.0875 129.9125) (end 142.0875 128.80625) (width 0.2) (layer "F.Cu") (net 5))
 (segment (start 152.103 138.1625) (end 151.526 138.1625) (width 0.2) (layer "F.Cu") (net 5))
 (segment (start 142.0875 128.80625) (end 145.78125 132.5) (width 0.2) (layer "F.Cu") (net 5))
 (segment (start 150.7615 132.75) (end 153.7385 132.75) (width 0.2) (layer "F.Cu") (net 5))
 (segment (start 152.8635 135.6625) (end 151.774 135.6625) (width 0.2) (layer "F.Cu") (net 5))
 (segment (start 150.3875 134.276) (end 150.3875 133.124) (width 0.2) (layer "F.Cu") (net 5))
 (via (at 146.25 132.5) (size 0.6) (drill 0.3) (layers "F.Cu" "B.Cu") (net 5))
 (via (at 149.5 133) (size 0.6) (drill 0.3) (layers "F.Cu" "B.Cu") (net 5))
 (segment (start 146.75 133) (end 149.5 133) (width 0.2) (layer "B.Cu") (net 5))
 (segment (start 146.25 132.5) (end 146.75 133) (width 0.2) (layer "B.Cu") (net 5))
 (segment (start 147.436 139.54) (end 147.8135 139.1625) (width 0.2) (layer "F.Cu") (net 13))
 (segment (start 128.5 127.546999) (end 140.493001 139.54) (width 0.2) (layer "F.Cu") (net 13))
 (segment (start 143 139.54) (end 147.436 139.54) (width 0.2) (layer "F.Cu") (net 13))
 (segment (start 140.493001 139.54) (end 143 139.54) (width 0.2) (layer "F.Cu") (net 13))
 (segment (start 128.5 125) (end 128.5 127.546999) (width 0.2) (layer "F.Cu") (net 13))
 (segment (start 140.5 137) (end 135.25 131.75) (width 0.2) (layer "F.Cu") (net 14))
 (segment (start 147.676 132.324) (end 143 137) (width 0.2) (layer "F.Cu") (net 14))
 (segment (start 147.676 131.8) (end 147.676 132.324) (width 0.2) (layer "F.Cu") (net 14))
 (segment (start 143 137) (end 140.5 137) (width 0.2) (layer "F.Cu") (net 14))
 (segment (start 145.218134 126.10625) (end 146.276 127.164116) (width 0.2) (layer "F.Cu") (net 10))
 (segment (start 143.9125 128.80625) (end 144.8375 128.80625) (width 0.2) (layer "F.Cu") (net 10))
 (segment (start 143.95 125.55625) (end 144.5 126.10625) (width 0.2) (layer "F.Cu") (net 10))
 (segment (start 146.276 128.69275) (end 145.5 129.46875) (width 0.2) (layer "F.Cu") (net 10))
 (segment (start 144.8375 128.80625) (end 145.5 129.46875) (width 0.2) (layer "F.Cu") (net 10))
 (segment (start 144.5 126.10625) (end 145.218134 126.10625) (width 0.2) (layer "F.Cu") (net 10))
 (segment (start 146.276 127.164116) (end 146.276 128.69275) (width 0.2) (layer "F.Cu") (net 10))
 (segment (start 152.043134 141.4385) (end 152.476 141.005634) (width 0.2) (layer "F.Cu") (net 16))
 (segment (start 150.575 140.929634) (end 151.083866 141.4385) (width 0.2) (layer "F.Cu") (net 16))
 (segment (start 150.101 137.9385) (end 150.575 138.4125) (width 0.2) (layer "F.Cu") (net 16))
 (segment (start 148.75 136.551) (end 148.75 137.629634) (width 0.2) (layer "F.Cu") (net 16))
 (segment (start 148.75 137.629634) (end 149.058866 137.9385) (width 0.2) (layer "F.Cu") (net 16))
 (segment (start 151.083866 141.4385) (end 152.043134 141.4385) (width 0.2) (layer "F.Cu") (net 16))
 (segment (start 152.476 141.005634) (end 152.476 139.6625) (width 0.2) (layer "F.Cu") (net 16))
 (segment (start 149.6385 135.6625) (end 148.75 136.551) (width 0.2) (layer "F.Cu") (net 16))
 (segment (start 153.026 139.1125) (end 153.926 139.1125) (width 0.2) (layer "F.Cu") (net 16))
 (segment (start 150.575 138.4125) (end 150.575 140.929634) (width 0.2) (layer "F.Cu") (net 16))
 (segment (start 152.476 139.6625) (end 153.026 139.1125) (width 0.2) (layer "F.Cu") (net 16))
 (segment (start 149.058866 137.9385) (end 150.101 137.9385) (width 0.2) (layer "F.Cu") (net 16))
 (segment (start 155.426 131.8) (end 153.7385 131.8) (width 0.2) (layer "F.Cu") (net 6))
 (segment (start 151.5635 139.15) (end 151.526 139.1125) (width 0.2) (layer "F.Cu") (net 17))
 (segment (start 151.5635 140.6625) (end 151.5635 139.15) (width 0.2) (layer "F.Cu") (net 17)))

